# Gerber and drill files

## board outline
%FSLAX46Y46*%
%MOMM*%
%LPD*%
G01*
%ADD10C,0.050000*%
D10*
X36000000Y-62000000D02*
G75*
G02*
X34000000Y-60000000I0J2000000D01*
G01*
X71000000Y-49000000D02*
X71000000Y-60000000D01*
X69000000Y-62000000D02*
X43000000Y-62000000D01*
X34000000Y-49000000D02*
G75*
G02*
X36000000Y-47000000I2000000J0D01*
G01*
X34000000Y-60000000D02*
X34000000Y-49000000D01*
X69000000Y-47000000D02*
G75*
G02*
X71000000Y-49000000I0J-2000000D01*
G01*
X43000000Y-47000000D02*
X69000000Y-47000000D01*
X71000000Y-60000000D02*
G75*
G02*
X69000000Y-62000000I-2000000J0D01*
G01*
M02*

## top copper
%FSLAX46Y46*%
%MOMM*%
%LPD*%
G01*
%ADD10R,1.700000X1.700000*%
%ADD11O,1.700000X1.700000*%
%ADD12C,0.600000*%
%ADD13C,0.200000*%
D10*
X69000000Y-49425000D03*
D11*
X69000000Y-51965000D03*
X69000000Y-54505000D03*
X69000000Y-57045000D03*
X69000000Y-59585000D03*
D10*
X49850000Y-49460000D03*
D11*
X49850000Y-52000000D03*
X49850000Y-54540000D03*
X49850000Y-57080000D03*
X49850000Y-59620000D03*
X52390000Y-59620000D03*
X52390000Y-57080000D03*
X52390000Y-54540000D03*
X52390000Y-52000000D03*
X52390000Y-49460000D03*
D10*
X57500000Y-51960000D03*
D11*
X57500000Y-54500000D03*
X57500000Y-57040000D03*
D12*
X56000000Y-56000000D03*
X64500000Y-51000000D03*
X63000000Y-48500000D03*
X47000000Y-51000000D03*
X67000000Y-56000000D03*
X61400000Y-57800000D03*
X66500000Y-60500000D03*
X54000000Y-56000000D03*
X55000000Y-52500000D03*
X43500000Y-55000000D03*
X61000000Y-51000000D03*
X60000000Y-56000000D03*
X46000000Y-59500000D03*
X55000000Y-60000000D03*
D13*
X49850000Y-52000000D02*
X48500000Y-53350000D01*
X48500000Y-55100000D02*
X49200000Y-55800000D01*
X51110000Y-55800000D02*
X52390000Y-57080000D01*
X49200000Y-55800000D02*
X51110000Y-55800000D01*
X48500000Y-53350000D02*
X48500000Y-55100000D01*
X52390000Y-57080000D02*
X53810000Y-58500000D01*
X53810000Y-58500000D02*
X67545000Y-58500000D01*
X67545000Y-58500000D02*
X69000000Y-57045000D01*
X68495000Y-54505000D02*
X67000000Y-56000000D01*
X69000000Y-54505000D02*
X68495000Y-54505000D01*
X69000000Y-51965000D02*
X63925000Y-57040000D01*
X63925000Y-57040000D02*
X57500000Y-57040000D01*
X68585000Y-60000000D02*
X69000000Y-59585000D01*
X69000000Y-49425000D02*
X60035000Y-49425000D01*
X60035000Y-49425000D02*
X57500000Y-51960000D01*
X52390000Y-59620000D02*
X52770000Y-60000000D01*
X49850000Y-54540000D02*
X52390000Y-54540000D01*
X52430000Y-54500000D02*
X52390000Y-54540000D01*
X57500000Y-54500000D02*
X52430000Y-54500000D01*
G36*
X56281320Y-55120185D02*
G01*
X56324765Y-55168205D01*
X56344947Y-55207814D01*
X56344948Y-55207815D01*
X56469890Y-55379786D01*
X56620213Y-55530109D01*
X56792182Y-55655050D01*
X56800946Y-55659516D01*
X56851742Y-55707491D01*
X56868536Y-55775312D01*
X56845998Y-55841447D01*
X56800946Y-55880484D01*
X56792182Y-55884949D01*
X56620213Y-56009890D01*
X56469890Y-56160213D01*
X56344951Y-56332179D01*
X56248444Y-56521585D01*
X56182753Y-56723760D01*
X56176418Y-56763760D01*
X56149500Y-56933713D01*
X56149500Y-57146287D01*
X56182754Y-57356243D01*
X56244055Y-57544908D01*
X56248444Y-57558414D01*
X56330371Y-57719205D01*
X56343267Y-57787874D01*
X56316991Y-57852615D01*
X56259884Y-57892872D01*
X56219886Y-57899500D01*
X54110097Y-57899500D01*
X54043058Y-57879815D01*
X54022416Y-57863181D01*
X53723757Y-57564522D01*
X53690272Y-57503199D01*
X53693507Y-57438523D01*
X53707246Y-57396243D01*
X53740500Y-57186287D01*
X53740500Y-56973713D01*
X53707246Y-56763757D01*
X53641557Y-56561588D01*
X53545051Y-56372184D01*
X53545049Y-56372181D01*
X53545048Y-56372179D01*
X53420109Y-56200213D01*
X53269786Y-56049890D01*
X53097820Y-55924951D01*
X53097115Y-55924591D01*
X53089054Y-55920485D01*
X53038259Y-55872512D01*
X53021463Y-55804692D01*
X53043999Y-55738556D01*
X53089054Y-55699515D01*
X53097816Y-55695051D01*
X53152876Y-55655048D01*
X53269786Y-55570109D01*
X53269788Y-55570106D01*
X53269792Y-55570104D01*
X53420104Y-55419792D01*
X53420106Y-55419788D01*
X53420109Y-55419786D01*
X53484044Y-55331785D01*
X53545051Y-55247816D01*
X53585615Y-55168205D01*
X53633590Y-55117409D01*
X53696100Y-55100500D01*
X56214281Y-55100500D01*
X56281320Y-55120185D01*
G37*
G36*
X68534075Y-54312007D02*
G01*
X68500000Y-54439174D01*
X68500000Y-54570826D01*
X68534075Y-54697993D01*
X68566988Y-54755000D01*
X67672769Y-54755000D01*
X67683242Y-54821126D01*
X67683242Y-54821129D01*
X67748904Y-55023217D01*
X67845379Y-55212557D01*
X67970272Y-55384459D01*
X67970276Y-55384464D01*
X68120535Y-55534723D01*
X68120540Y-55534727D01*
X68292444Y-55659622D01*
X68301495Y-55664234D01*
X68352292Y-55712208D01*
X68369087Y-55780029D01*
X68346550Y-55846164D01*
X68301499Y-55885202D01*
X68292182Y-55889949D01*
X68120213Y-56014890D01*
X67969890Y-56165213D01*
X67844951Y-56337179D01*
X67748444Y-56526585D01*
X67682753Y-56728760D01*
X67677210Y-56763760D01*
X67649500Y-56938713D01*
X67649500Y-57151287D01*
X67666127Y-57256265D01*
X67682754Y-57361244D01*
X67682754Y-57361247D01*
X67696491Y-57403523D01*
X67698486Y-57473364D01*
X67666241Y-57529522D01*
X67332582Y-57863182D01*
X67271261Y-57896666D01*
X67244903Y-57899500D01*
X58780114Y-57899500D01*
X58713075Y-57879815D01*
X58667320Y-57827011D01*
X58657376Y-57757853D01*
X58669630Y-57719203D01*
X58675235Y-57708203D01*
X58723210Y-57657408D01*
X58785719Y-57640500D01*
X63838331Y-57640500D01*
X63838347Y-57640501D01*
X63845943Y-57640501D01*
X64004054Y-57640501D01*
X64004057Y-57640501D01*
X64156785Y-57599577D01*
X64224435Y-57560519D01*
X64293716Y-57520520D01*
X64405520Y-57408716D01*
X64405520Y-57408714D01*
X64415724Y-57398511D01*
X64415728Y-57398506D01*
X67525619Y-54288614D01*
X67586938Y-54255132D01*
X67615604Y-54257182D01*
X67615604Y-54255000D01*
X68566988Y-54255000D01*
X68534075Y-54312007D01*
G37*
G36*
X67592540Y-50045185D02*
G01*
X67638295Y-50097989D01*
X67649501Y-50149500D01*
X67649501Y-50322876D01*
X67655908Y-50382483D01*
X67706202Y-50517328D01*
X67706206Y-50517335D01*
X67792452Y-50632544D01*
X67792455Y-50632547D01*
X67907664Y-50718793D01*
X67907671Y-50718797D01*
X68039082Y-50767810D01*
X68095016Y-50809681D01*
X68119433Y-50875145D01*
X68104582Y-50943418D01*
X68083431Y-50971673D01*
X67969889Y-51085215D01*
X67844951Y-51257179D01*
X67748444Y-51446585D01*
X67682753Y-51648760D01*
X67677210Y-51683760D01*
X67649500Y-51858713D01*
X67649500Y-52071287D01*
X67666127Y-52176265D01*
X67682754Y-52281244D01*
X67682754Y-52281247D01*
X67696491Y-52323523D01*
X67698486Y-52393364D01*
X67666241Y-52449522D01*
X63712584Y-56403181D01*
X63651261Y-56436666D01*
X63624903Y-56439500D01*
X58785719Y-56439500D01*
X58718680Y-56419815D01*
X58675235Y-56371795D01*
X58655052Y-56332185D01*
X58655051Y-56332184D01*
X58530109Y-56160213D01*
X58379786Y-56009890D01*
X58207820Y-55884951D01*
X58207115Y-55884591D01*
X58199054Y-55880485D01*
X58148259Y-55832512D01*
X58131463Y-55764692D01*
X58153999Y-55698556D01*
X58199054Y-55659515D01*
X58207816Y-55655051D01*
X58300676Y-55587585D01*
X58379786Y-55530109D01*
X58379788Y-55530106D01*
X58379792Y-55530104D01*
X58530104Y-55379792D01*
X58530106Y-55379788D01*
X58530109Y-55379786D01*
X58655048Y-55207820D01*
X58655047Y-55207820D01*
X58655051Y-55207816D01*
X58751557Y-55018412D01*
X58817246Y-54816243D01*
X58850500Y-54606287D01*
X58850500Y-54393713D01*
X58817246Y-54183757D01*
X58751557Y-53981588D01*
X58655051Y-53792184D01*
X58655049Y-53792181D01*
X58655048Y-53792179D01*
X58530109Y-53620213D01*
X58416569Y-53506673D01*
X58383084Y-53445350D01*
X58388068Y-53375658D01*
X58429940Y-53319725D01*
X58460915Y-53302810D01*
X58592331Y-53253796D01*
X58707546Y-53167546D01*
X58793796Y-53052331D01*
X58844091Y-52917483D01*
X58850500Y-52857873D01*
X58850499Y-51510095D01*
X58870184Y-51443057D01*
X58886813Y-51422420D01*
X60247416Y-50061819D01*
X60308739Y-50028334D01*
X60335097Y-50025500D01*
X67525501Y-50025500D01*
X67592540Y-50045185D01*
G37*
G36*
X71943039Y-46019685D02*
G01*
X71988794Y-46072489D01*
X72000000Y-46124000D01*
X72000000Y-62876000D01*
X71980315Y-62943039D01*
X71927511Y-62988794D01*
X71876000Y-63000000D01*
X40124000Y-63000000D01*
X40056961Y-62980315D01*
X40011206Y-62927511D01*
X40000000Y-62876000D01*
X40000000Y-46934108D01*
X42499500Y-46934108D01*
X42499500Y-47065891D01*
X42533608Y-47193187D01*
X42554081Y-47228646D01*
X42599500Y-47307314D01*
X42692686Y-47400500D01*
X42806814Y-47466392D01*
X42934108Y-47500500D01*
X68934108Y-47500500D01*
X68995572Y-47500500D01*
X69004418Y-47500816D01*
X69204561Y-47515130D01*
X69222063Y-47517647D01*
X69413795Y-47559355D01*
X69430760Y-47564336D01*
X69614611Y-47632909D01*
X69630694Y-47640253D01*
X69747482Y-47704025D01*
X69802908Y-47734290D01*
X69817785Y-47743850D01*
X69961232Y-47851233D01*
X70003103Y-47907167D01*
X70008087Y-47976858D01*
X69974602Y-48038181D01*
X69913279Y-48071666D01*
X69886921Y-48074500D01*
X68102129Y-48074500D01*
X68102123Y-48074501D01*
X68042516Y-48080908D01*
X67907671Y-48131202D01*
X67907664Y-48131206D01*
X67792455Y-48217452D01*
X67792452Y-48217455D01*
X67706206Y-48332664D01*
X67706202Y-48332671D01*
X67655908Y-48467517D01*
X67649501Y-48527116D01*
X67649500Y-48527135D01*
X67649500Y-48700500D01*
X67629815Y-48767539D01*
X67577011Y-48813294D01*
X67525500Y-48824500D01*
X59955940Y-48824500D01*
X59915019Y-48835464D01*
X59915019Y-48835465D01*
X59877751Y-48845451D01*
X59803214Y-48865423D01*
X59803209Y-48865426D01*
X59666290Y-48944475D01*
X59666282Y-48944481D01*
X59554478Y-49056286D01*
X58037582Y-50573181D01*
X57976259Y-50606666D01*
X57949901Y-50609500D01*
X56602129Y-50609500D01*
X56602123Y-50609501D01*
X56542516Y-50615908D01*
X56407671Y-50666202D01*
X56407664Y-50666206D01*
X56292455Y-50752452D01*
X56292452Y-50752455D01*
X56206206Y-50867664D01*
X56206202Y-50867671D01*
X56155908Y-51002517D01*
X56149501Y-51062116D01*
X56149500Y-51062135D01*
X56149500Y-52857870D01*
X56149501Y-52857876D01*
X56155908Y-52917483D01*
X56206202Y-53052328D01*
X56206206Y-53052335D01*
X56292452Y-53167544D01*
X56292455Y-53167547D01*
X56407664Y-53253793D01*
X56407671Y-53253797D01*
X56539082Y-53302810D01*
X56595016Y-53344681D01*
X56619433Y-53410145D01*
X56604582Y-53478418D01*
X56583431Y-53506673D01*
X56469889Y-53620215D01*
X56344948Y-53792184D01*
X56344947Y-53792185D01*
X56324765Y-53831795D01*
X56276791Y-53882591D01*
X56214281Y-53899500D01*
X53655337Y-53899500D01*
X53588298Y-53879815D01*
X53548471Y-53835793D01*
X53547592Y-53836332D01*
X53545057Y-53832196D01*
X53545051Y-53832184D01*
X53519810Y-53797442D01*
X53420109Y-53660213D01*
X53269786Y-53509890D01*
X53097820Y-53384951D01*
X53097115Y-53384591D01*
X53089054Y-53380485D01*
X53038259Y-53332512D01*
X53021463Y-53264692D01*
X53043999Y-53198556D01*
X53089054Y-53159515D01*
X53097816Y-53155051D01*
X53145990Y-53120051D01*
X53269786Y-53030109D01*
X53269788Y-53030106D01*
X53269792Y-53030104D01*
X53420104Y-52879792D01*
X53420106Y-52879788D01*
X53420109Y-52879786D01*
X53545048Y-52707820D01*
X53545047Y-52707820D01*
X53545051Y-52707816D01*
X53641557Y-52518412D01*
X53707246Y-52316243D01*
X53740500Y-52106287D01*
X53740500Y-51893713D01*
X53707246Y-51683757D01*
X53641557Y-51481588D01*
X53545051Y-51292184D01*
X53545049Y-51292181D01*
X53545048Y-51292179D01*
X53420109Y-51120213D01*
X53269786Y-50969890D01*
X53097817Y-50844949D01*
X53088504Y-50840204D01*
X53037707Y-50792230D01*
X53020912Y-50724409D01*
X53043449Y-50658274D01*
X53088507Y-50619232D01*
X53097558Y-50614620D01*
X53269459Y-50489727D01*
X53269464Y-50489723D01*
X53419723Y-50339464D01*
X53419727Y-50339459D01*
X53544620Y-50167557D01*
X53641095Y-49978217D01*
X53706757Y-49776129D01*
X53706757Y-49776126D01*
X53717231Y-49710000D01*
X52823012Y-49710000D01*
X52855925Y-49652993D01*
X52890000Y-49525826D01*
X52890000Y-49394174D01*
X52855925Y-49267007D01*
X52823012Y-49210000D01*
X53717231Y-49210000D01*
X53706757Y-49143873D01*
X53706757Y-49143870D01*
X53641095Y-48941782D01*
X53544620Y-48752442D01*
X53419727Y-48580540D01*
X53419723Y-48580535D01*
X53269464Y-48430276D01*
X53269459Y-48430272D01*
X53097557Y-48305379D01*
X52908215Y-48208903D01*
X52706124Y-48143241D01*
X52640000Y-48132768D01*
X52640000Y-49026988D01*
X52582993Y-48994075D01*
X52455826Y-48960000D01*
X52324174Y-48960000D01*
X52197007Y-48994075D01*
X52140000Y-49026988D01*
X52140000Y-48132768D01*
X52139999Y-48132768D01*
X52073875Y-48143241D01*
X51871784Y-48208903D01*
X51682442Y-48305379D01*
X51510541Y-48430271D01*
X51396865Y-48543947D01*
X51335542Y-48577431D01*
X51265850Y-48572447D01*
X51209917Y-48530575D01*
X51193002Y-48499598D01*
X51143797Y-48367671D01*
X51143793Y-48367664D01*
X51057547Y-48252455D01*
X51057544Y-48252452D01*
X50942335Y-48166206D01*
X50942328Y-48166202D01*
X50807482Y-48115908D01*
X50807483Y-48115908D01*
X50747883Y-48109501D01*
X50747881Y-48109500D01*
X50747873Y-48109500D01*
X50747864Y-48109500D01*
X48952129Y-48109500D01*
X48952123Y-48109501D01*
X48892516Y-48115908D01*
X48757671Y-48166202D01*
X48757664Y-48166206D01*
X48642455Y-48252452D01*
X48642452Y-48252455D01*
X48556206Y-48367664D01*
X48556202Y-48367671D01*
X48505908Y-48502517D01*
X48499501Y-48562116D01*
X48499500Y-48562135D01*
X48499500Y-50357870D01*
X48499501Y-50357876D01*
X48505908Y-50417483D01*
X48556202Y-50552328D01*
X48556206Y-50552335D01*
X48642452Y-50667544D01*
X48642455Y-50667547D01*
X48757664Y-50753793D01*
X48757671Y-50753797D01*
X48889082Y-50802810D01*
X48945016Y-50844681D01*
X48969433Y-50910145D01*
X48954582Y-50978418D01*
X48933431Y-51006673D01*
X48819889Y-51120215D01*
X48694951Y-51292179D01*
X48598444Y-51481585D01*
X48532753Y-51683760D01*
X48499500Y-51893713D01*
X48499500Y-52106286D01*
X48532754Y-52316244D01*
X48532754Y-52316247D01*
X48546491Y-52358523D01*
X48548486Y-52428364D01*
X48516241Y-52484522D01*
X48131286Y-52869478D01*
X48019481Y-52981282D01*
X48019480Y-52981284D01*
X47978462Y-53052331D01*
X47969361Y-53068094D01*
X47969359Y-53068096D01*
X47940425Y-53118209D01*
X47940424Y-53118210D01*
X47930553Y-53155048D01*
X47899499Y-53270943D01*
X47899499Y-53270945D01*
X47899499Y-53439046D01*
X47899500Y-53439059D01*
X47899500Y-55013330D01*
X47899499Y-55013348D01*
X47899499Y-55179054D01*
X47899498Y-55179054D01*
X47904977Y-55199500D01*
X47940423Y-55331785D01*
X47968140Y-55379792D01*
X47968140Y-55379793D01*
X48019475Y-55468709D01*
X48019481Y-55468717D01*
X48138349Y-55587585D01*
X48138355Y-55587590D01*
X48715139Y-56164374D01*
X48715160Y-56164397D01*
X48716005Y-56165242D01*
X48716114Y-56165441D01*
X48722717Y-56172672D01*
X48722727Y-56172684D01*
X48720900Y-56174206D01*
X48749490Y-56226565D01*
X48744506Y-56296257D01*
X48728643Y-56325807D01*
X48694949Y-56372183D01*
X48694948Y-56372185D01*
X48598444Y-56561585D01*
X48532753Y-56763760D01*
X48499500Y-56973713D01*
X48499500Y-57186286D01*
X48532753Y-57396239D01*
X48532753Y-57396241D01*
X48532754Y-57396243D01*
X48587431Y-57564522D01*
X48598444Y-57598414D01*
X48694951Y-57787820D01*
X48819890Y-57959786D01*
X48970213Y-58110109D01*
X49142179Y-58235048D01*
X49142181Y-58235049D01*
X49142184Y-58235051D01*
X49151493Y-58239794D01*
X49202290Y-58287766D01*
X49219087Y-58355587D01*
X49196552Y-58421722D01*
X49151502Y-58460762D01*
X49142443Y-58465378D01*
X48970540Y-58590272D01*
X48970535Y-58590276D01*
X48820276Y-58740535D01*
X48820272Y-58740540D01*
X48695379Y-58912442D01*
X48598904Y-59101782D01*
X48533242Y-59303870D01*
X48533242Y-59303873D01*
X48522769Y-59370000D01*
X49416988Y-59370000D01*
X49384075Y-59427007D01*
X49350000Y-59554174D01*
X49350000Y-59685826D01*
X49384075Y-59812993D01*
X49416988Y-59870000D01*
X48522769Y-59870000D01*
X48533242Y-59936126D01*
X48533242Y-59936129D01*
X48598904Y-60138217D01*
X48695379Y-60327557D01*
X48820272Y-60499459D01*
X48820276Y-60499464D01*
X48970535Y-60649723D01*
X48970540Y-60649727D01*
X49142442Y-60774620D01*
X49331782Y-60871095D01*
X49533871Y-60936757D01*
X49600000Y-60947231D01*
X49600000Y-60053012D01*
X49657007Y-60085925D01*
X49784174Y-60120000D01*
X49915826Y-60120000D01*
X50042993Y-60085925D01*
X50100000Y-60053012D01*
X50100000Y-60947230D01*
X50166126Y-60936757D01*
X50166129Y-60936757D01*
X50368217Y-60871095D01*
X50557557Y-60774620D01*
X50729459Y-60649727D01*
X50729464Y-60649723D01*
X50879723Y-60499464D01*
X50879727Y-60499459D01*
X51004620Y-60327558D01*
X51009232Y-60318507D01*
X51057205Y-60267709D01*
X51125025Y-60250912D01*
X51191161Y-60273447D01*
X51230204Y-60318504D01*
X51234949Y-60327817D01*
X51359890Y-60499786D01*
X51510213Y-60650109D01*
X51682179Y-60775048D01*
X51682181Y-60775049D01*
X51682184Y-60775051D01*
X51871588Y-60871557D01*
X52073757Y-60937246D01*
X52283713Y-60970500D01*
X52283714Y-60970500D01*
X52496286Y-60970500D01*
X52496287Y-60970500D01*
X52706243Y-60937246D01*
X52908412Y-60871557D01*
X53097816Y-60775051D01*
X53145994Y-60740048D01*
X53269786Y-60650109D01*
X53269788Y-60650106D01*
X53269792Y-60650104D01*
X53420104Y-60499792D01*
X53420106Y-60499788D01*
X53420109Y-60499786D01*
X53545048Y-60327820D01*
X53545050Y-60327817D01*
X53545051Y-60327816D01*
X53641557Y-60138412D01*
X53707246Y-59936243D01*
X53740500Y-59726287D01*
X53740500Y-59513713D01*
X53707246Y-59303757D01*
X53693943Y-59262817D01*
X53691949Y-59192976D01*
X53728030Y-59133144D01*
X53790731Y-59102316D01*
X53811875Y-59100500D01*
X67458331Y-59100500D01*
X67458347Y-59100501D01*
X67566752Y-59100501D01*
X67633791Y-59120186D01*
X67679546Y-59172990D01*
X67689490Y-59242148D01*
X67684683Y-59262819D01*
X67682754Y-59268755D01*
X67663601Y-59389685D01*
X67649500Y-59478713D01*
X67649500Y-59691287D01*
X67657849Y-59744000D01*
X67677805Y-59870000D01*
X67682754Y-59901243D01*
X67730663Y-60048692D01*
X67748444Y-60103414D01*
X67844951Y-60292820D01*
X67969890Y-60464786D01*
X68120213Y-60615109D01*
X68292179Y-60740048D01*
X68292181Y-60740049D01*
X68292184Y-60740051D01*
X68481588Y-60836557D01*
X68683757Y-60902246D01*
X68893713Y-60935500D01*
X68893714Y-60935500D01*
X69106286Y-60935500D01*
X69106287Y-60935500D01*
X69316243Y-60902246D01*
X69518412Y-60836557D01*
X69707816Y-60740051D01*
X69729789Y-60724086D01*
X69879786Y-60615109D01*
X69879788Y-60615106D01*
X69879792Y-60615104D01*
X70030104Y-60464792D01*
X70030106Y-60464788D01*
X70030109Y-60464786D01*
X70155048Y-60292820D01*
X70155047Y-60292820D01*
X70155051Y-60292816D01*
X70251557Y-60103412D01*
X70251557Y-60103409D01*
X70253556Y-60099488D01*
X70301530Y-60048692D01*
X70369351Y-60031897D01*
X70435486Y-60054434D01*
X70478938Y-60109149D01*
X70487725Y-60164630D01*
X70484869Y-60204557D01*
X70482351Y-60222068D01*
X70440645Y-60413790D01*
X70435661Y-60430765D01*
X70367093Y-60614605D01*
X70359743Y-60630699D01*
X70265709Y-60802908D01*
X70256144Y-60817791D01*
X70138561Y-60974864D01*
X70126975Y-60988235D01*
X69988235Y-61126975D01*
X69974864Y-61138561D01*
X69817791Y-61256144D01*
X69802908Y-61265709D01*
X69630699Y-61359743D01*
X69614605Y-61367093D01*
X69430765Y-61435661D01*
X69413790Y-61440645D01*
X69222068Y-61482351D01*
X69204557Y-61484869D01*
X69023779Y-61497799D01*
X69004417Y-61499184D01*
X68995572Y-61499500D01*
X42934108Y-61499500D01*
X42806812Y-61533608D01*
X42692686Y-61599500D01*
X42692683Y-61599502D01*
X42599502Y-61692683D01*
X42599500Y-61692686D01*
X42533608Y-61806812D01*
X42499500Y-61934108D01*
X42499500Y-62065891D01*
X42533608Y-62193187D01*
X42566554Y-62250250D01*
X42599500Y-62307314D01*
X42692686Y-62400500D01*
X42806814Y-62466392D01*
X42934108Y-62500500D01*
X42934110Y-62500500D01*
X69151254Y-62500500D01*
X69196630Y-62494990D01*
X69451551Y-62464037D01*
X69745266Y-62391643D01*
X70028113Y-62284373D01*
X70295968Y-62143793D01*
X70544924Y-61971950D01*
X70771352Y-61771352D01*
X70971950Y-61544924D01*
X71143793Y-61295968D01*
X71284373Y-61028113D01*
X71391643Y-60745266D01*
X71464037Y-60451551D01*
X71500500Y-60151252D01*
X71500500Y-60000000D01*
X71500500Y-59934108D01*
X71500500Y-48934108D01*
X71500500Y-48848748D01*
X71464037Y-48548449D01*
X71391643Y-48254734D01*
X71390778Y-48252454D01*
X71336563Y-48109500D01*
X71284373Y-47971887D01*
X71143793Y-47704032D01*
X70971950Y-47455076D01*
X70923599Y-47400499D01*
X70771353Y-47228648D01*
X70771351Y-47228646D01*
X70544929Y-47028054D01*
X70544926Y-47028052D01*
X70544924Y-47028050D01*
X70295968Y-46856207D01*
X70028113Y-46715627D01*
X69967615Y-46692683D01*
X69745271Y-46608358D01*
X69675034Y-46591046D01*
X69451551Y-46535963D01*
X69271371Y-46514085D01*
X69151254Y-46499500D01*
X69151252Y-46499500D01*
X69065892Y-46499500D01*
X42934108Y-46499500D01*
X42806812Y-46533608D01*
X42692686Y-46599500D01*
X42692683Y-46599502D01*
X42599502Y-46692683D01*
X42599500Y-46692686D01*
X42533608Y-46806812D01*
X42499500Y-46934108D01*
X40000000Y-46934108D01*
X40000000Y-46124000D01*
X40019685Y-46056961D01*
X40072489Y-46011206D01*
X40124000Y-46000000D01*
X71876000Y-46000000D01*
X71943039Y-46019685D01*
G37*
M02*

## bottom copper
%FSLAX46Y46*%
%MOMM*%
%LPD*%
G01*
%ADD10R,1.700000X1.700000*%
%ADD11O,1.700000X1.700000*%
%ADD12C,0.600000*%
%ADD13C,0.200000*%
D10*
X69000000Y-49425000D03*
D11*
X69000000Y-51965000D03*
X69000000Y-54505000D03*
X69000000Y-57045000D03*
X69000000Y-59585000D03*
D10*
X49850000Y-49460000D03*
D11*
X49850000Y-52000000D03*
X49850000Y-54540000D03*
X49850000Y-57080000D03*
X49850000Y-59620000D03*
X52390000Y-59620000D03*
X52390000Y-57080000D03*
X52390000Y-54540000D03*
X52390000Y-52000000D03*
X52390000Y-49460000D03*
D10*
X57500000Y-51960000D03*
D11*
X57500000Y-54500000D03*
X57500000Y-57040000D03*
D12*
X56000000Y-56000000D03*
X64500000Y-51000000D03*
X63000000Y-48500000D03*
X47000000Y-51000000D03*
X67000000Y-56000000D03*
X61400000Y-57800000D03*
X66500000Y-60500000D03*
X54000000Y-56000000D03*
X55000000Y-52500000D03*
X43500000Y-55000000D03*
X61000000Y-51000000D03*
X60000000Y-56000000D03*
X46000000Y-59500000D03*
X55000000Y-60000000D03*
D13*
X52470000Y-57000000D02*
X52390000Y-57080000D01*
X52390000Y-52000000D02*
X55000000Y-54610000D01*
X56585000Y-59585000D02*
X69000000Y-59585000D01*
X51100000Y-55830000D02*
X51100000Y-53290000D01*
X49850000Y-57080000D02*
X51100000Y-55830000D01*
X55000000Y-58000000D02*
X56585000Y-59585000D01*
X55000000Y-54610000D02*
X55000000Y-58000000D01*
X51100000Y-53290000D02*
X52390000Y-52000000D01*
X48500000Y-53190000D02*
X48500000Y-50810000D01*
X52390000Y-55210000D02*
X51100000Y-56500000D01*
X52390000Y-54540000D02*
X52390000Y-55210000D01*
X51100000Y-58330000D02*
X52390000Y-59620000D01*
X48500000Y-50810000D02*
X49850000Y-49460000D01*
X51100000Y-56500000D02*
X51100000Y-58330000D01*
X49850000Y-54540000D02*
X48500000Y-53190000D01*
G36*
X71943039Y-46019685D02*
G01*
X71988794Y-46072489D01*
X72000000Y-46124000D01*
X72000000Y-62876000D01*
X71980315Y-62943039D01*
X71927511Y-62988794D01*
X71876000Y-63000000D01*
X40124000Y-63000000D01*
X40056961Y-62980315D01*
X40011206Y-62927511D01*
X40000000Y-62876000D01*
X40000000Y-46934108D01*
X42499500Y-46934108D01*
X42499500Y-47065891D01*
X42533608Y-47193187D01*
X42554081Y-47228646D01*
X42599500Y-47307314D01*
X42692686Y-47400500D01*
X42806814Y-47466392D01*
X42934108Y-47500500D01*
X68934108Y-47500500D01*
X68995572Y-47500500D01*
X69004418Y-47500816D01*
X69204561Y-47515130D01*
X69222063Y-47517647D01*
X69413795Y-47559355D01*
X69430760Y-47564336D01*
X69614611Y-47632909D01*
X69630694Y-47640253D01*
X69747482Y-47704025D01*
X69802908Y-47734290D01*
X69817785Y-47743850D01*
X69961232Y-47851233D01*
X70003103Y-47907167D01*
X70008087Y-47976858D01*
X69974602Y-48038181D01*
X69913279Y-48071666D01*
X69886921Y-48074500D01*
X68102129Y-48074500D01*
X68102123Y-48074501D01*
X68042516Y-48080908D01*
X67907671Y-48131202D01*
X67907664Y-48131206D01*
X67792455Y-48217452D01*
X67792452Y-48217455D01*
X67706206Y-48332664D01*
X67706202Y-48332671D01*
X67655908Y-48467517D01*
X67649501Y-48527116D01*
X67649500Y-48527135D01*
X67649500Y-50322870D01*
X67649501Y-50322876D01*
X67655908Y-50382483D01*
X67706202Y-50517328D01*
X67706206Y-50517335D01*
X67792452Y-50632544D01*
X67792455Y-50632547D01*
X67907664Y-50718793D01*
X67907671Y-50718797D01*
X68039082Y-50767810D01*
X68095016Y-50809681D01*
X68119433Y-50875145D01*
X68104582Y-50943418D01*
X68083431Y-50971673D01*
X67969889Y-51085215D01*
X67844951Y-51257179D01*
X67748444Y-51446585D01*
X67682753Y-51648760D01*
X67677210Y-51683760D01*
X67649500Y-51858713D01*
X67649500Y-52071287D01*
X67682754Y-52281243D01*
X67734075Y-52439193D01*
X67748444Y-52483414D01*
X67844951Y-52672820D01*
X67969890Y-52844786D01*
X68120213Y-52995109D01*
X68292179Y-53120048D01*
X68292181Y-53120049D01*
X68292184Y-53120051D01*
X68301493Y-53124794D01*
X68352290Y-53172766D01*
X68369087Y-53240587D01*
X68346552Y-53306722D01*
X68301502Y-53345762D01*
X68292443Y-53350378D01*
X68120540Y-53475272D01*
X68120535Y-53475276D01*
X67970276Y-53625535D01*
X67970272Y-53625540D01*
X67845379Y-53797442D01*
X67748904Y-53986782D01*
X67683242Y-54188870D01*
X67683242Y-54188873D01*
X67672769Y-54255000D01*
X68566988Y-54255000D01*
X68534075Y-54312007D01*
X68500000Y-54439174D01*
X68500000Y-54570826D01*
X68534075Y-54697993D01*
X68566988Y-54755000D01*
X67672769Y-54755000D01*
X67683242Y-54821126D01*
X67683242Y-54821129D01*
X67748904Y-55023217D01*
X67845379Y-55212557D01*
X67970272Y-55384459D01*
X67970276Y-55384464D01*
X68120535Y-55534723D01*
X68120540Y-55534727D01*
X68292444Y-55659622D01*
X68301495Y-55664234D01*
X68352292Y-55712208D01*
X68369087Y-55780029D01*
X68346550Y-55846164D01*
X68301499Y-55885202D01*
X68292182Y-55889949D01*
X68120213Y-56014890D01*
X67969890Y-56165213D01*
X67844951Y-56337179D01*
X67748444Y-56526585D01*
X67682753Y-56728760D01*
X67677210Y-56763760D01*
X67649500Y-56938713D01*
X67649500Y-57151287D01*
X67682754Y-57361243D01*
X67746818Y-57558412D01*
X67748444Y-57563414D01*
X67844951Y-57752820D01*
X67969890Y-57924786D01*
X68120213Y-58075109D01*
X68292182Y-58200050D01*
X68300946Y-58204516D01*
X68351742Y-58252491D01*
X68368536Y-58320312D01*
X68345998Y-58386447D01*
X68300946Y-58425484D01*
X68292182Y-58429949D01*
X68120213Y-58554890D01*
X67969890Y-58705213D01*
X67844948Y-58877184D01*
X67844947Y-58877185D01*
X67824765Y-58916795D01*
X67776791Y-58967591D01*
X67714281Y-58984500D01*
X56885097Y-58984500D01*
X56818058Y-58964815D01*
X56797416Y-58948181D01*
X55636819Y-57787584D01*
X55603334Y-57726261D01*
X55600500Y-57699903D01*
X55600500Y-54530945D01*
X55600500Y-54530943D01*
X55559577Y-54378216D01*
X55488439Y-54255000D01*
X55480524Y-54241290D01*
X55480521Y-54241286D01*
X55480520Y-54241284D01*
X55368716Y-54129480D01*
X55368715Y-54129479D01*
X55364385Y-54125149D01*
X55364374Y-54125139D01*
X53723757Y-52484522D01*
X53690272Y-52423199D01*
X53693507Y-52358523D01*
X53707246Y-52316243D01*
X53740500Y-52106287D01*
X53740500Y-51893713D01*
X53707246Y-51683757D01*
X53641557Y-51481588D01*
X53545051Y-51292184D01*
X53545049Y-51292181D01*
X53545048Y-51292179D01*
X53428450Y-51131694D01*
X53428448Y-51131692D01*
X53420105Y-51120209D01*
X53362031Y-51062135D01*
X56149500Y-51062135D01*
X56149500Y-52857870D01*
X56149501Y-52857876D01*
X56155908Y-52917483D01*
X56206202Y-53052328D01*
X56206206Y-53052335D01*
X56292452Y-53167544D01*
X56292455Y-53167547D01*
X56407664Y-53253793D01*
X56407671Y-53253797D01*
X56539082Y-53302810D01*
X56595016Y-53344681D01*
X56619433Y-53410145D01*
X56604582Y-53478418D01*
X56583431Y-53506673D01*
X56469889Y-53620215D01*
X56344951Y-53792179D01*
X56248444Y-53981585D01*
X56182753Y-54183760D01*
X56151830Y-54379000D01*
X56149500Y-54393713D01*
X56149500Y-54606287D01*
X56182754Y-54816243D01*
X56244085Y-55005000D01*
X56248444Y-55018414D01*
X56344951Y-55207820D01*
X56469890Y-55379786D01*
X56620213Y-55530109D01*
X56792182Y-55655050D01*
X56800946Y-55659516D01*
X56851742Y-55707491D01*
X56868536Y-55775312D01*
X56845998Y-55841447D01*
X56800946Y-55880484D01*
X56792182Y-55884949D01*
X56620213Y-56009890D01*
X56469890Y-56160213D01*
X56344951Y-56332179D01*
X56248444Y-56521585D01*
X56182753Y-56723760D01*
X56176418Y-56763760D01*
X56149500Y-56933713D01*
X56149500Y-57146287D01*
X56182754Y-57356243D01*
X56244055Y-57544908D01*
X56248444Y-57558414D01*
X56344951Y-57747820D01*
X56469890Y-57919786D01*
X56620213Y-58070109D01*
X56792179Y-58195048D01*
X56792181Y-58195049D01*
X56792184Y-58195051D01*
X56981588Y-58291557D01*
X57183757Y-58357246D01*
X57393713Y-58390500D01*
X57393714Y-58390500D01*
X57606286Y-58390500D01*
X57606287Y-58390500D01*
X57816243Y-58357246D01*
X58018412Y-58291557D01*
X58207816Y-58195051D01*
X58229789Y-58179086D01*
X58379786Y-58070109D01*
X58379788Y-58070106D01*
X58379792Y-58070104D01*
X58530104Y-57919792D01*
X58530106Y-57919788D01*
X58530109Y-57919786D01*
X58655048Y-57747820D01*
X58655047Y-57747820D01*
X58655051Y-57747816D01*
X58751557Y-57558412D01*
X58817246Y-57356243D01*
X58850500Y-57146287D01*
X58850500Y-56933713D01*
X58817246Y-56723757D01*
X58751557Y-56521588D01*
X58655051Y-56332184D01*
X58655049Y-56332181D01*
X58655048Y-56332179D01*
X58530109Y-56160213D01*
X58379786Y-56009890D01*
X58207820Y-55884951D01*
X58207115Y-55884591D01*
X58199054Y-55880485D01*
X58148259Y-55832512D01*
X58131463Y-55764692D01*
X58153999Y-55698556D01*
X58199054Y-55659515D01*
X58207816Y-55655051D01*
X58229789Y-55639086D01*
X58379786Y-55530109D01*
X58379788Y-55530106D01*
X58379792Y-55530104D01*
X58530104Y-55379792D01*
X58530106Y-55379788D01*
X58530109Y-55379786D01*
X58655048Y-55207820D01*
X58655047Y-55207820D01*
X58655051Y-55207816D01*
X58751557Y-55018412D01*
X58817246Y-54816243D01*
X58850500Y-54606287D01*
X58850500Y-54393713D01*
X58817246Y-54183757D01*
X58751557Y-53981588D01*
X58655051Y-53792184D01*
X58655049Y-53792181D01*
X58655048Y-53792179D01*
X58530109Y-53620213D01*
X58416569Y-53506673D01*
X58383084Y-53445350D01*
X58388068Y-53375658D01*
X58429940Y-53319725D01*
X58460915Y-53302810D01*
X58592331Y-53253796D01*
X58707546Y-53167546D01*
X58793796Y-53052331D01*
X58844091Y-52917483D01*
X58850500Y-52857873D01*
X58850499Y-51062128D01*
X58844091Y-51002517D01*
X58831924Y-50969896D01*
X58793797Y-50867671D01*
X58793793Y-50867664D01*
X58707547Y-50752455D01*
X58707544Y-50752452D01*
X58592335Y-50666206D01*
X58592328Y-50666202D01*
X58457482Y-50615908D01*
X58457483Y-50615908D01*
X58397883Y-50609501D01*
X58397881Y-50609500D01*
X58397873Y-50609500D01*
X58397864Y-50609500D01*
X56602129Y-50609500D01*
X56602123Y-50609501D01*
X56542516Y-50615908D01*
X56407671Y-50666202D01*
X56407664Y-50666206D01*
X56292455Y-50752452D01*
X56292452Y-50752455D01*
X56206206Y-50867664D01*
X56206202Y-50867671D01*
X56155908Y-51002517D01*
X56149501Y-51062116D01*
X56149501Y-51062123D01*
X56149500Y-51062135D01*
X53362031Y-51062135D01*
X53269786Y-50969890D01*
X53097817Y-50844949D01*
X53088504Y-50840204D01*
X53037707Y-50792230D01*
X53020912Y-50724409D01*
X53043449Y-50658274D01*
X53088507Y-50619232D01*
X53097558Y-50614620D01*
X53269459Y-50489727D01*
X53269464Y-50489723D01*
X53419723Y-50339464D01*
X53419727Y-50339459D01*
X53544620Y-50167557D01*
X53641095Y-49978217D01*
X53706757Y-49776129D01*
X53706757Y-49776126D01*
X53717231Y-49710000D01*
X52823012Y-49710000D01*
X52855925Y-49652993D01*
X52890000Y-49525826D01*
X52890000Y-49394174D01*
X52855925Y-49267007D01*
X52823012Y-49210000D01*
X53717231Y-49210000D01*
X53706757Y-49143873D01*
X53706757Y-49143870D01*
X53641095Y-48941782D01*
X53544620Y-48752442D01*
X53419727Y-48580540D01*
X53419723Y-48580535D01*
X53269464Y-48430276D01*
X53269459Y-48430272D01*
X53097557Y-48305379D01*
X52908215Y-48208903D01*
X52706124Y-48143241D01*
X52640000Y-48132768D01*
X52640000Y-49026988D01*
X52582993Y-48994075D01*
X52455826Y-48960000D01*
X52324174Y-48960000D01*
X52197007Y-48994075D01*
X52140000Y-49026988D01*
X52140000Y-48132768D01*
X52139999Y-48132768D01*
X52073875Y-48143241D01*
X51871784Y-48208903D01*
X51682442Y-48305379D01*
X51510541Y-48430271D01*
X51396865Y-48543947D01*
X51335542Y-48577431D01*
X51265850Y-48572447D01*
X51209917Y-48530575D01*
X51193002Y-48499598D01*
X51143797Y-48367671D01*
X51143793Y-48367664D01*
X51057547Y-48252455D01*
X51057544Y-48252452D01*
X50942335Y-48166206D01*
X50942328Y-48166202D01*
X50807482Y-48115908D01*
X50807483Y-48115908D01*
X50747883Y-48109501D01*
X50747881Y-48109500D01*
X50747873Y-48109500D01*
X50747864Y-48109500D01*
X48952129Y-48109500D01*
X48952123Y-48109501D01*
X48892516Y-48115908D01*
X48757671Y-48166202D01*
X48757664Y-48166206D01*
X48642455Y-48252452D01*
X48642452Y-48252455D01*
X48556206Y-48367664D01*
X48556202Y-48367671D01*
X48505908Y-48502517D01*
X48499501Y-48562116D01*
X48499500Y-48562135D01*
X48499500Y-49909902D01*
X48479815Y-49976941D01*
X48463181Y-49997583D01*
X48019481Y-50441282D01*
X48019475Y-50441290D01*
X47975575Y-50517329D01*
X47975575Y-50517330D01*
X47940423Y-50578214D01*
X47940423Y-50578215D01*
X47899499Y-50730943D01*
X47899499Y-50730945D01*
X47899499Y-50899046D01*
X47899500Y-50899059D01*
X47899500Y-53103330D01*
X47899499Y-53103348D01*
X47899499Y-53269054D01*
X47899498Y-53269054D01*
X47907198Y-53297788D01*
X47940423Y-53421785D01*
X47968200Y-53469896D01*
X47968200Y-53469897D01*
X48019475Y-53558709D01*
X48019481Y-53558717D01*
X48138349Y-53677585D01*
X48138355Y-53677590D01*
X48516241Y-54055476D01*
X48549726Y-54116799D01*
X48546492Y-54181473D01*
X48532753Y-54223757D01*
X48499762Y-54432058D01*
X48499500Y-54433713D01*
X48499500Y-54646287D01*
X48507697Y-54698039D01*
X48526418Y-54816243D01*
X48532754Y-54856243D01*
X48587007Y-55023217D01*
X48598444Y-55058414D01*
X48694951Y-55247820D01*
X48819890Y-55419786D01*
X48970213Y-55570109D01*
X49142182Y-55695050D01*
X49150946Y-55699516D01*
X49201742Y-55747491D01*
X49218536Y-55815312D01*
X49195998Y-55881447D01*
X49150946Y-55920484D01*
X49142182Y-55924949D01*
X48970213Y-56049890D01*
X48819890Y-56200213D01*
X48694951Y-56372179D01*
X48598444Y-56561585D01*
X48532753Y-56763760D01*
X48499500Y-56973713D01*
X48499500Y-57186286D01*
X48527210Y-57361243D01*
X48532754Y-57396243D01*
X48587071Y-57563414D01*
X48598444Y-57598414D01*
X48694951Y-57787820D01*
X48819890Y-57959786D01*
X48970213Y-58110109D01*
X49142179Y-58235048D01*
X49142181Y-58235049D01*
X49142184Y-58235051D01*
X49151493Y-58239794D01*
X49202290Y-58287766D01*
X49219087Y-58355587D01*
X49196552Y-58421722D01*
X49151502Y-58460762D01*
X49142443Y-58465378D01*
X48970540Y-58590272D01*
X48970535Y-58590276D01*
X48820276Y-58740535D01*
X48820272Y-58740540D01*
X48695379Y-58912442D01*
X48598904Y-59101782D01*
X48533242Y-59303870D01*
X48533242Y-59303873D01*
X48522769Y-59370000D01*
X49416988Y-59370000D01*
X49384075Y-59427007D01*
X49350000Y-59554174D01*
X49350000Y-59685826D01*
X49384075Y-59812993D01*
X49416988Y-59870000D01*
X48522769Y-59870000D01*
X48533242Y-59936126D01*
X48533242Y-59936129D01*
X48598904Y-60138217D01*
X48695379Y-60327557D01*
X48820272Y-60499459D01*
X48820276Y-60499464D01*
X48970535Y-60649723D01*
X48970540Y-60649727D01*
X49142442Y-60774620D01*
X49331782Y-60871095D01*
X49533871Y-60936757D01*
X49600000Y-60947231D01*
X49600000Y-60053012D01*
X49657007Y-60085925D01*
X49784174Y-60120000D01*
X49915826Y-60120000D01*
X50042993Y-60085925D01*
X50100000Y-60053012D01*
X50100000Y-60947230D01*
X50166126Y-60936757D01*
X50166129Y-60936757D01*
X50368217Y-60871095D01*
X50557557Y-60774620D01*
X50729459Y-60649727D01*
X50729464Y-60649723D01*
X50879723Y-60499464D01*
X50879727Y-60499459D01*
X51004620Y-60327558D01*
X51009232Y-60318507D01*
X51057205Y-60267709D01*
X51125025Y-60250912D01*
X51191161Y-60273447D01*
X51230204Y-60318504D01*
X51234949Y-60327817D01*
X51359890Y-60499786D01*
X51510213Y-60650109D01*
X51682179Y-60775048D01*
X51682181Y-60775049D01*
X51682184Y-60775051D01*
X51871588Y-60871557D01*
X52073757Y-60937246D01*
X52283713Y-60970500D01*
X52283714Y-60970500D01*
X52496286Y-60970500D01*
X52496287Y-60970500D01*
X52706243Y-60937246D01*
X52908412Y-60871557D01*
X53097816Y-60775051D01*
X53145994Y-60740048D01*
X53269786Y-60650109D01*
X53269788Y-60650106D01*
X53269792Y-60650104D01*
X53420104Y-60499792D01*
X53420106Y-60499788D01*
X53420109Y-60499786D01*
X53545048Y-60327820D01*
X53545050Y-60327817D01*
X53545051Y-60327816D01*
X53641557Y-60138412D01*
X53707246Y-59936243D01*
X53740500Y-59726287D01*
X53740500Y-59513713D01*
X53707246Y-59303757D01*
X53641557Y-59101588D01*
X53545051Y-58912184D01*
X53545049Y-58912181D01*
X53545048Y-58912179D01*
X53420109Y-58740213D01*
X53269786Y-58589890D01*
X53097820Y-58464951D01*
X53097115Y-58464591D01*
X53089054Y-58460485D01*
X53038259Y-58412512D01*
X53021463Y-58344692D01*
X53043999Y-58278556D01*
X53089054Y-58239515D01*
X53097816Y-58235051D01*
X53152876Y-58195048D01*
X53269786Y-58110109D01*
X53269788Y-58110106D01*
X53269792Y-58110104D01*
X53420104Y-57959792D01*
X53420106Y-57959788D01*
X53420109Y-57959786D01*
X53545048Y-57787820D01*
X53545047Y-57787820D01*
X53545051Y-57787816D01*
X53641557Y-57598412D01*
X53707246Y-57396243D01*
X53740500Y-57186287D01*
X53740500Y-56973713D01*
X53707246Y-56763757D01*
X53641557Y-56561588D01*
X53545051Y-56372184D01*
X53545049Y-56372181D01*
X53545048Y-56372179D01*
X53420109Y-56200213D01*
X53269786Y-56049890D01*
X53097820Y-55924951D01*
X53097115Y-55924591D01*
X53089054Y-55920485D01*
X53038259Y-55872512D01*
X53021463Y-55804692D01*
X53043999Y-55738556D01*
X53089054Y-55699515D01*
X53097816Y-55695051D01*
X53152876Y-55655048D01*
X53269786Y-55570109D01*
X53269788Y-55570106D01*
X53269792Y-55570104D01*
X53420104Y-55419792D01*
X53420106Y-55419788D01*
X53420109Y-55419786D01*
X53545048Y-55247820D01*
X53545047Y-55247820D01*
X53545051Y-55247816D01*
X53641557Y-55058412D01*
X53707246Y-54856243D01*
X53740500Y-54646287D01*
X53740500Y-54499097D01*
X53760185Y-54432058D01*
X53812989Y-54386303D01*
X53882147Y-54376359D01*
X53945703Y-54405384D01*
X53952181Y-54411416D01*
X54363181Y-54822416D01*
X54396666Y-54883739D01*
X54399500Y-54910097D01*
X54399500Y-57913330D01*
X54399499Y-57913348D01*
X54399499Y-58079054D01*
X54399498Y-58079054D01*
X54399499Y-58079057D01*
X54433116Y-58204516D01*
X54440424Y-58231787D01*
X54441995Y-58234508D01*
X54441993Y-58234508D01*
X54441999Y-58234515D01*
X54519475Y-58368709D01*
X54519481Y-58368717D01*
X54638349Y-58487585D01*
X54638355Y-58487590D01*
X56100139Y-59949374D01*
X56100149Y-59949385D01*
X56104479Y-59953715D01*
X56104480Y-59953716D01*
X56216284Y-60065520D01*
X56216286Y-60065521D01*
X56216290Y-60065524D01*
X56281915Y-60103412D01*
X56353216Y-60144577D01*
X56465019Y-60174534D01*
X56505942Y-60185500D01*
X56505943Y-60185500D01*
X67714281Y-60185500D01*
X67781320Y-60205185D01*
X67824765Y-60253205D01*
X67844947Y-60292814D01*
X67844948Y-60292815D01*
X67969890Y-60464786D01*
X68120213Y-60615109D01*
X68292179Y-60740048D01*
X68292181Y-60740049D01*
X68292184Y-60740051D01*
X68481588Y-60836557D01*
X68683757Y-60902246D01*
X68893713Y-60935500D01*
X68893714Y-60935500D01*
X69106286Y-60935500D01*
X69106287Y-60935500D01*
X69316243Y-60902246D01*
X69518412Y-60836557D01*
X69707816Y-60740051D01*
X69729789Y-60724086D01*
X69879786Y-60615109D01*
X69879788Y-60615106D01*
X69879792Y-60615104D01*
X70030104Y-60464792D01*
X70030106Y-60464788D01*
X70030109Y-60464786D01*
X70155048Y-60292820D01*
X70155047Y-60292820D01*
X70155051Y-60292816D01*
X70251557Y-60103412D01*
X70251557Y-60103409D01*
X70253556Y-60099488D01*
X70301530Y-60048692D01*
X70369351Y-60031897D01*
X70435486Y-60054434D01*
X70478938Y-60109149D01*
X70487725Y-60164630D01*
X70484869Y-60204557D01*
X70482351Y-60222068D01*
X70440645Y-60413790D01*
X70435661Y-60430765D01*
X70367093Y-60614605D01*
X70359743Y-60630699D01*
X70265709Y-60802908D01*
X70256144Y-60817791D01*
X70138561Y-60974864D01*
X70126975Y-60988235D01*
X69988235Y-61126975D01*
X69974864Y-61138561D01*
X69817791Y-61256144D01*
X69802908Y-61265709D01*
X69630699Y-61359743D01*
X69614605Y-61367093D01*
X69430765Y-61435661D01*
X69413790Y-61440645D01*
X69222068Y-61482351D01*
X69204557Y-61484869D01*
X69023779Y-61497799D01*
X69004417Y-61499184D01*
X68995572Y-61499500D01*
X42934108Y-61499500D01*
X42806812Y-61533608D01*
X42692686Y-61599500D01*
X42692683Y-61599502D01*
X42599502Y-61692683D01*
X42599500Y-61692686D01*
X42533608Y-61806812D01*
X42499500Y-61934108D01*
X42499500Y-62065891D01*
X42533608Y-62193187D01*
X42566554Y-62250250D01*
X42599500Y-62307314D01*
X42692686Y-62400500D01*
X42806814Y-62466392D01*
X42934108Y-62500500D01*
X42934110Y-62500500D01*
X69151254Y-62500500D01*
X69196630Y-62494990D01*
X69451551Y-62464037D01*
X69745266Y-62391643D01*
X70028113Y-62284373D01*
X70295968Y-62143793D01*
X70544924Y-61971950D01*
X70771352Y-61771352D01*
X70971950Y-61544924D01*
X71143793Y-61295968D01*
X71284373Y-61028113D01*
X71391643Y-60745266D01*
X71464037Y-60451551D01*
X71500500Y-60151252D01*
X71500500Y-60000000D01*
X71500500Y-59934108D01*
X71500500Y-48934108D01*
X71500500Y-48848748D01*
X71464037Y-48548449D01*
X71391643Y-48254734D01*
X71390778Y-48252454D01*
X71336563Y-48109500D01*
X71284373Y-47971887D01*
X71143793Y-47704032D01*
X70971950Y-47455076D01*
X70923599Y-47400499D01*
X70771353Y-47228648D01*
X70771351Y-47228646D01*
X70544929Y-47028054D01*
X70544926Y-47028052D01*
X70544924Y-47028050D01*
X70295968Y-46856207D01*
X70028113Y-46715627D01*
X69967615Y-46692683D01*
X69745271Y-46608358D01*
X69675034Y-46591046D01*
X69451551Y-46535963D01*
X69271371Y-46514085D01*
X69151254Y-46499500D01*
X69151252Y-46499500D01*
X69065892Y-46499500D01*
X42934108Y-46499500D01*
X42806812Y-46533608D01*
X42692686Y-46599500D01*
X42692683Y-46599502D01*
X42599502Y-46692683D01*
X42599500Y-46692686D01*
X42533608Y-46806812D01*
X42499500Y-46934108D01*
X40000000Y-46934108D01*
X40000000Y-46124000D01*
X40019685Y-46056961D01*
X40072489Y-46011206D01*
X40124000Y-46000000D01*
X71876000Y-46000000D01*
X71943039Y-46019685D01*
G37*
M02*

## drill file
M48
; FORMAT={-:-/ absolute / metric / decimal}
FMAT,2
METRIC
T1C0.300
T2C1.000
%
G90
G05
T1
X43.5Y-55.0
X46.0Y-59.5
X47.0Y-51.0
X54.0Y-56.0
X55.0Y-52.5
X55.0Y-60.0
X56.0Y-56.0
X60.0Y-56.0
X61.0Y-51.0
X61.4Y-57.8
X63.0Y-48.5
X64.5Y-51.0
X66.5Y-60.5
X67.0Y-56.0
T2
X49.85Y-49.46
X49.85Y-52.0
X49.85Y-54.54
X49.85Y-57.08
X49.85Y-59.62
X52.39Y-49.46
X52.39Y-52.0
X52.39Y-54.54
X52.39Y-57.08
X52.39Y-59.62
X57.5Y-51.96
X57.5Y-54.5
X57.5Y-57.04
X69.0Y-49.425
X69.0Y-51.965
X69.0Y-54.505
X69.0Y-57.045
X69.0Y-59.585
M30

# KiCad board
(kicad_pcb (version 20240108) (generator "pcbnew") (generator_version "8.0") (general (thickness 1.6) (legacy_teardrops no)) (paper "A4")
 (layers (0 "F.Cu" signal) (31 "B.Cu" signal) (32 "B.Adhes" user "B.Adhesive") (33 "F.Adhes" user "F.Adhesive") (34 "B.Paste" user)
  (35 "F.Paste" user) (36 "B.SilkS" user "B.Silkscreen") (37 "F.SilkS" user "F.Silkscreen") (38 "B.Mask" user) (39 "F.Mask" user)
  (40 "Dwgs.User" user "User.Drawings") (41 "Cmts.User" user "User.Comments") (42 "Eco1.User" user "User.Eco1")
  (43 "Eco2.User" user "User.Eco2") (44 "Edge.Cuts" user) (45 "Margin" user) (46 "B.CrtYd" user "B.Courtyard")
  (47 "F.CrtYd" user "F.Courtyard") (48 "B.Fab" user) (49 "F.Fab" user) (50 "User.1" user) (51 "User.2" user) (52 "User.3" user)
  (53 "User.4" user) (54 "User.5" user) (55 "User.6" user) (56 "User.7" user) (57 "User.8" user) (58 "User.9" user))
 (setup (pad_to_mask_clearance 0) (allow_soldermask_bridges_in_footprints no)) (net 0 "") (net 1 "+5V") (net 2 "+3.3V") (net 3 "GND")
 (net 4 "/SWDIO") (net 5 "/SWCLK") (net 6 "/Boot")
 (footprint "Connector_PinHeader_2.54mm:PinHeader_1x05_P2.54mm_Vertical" (layer "F.Cu") (at 69 49.425)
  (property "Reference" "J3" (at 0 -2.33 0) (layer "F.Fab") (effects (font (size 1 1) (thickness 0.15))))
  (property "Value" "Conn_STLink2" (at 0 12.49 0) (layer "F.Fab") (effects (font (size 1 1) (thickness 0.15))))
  (pad "1" thru_hole rect (at 0 0) (size 1.7 1.7) (drill 1) (layers "*.Cu" "*.Mask") (remove_unused_layers no) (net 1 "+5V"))
  (pad "2" thru_hole oval (at 0 2.54) (size 1.7 1.7) (drill 1) (layers "*.Cu" "*.Mask") (remove_unused_layers no) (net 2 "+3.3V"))
  (pad "3" thru_hole oval (at 0 5.08) (size 1.7 1.7) (drill 1) (layers "*.Cu" "*.Mask") (remove_unused_layers no) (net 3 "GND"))
  (pad "4" thru_hole oval (at 0 7.62) (size 1.7 1.7) (drill 1) (layers "*.Cu" "*.Mask") (remove_unused_layers no) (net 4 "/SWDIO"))
  (pad "5" thru_hole oval (at 0 10.16) (size 1.7 1.7) (drill 1) (layers "*.Cu" "*.Mask") (remove_unused_layers no) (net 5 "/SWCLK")))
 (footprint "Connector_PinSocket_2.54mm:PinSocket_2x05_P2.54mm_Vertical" (layer "F.Cu") (at 52.39 49.46)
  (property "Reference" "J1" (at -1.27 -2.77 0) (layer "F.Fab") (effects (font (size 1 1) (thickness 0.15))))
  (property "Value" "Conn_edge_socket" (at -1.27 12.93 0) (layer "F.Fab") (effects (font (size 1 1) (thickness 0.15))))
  (pad "1" thru_hole rect (at -2.54 0) (size 1.7 1.7) (drill 1) (layers "*.Cu" "*.Mask") (remove_unused_layers no) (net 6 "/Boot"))
  (pad "2" thru_hole oval (at -2.54 2.54) (size 1.7 1.7) (drill 1) (layers "*.Cu" "*.Mask") (remove_unused_layers no) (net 4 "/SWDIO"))
  (pad "3" thru_hole oval (at -2.54 5.08) (size 1.7 1.7) (drill 1) (layers "*.Cu" "*.Mask") (remove_unused_layers no) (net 6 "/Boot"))
  (pad "4" thru_hole oval (at -2.54 7.62) (size 1.7 1.7) (drill 1) (layers "*.Cu" "*.Mask") (remove_unused_layers no) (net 5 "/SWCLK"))
  (pad "5" thru_hole oval (at -2.54 10.16) (size 1.7 1.7) (drill 1) (layers "*.Cu" "*.Mask") (remove_unused_layers no) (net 3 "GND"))
  (pad "6" thru_hole oval (at 0 10.16) (size 1.7 1.7) (drill 1) (layers "*.Cu" "*.Mask") (remove_unused_layers no) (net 6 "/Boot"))
  (pad "7" thru_hole oval (at 0 7.62) (size 1.7 1.7) (drill 1) (layers "*.Cu" "*.Mask") (remove_unused_layers no) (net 4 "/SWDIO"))
  (pad "8" thru_hole oval (at 0 5.08) (size 1.7 1.7) (drill 1) (layers "*.Cu" "*.Mask") (remove_unused_layers no) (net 6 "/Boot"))
  (pad "9" thru_hole oval (at 0 2.54) (size 1.7 1.7) (drill 1) (layers "*.Cu" "*.Mask") (remove_unused_layers no) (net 5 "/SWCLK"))
  (pad "10" thru_hole oval (at 0 0) (size 1.7 1.7) (drill 1) (layers "*.Cu" "*.Mask") (remove_unused_layers no) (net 3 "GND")))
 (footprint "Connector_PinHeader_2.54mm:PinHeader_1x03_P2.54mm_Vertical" (layer "F.Cu") (at 57.5 51.96)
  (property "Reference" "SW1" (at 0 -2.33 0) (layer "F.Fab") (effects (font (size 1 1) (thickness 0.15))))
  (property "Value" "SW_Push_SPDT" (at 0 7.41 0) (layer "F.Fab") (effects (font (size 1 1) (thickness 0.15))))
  (pad "1" thru_hole rect (at 0 0) (size 1.7 1.7) (drill 1) (layers "*.Cu" "*.Mask") (remove_unused_layers no) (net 1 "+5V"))
  (pad "2" thru_hole oval (at 0 2.54) (size 1.7 1.7) (drill 1) (layers "*.Cu" "*.Mask") (remove_unused_layers no) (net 6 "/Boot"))
  (pad "3" thru_hole oval (at 0 5.08) (size 1.7 1.7) (drill 1) (layers "*.Cu" "*.Mask") (remove_unused_layers no) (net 2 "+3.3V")))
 (gr_arc (start 36 62) (mid 34.585786 61.414214) (end 34 60) (stroke (width 0.05) (type default)) (layer "Edge.Cuts"))
 (gr_line (start 71 49) (end 71 60) (stroke (width 0.05) (type default)) (layer "Edge.Cuts"))
 (gr_line (start 69 62) (end 43 62) (stroke (width 0.05) (type default)) (layer "Edge.Cuts"))
 (gr_arc (start 34 49) (mid 34.585786 47.585786) (end 36 47) (stroke (width 0.05) (type default)) (layer "Edge.Cuts"))
 (gr_line (start 34 60) (end 34 49) (stroke (width 0.05) (type default)) (layer "Edge.Cuts"))
 (gr_arc (start 69 47) (mid 70.414214 47.585786) (end 71 49) (stroke (width 0.05) (type default)) (layer "Edge.Cuts"))
 (gr_line (start 43 47) (end 69 47) (stroke (width 0.05) (type default)) (layer "Edge.Cuts"))
 (gr_arc (start 71 60) (mid 70.414214 61.414214) (end 69 62) (stroke (width 0.05) (type default)) (layer "Edge.Cuts"))
 (segment (start 49.85 52) (end 48.5 53.35) (width 0.2) (layer "F.Cu") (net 4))
 (segment (start 48.5 55.1) (end 49.2 55.8) (width 0.2) (layer "F.Cu") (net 4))
 (segment (start 51.11 55.8) (end 52.39 57.08) (width 0.2) (layer "F.Cu") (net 4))
 (segment (start 49.2 55.8) (end 51.11 55.8) (width 0.2) (layer "F.Cu") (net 4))
 (segment (start 48.5 53.35) (end 48.5 55.1) (width 0.2) (layer "F.Cu") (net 4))
 (segment (start 52.39 57.08) (end 53.81 58.5) (width 0.2) (layer "F.Cu") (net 4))
 (segment (start 53.81 58.5) (end 67.545 58.5) (width 0.2) (layer "F.Cu") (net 4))
 (segment (start 67.545 58.5) (end 69 57.045) (width 0.2) (layer "F.Cu") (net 4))
 (segment (start 52.47 57) (end 52.39 57.08) (width 0.2) (layer "B.Cu") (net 4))
 (segment (start 68.495 54.505) (end 67 56) (width 0.2) (layer "F.Cu") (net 3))
 (segment (start 69 54.505) (end 68.495 54.505) (width 0.2) (layer "F.Cu") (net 3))
 (via (at 56 56) (size 0.6) (drill 0.3) (layers "F.Cu" "B.Cu") (free yes) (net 3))
 (via (at 64.5 51) (size 0.6) (drill 0.3) (layers "F.Cu" "B.Cu") (free yes) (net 3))
 (via (at 63 48.5) (size 0.6) (drill 0.3) (layers "F.Cu" "B.Cu") (free yes) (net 3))
 (via (at 47 51) (size 0.6) (drill 0.3) (layers "F.Cu" "B.Cu") (free yes) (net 3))
 (via (at 67 56) (size 0.6) (drill 0.3) (layers "F.Cu" "B.Cu") (free yes) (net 3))
 (via (at 61.4 57.8) (size 0.6) (drill 0.3) (layers "F.Cu" "B.Cu") (free yes) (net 3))
 (via (at 66.5 60.5) (size 0.6) (drill 0.3) (layers "F.Cu" "B.Cu") (free yes) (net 3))
 (via (at 54 56) (size 0.6) (drill 0.3) (layers "F.Cu" "B.Cu") (free yes) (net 3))
 (via (at 55 52.5) (size 0.6) (drill 0.3) (layers "F.Cu" "B.Cu") (free yes) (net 3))
 (via (at 43.5 55) (size 0.6) (drill 0.3) (layers "F.Cu" "B.Cu") (free yes) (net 3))
 (via (at 61 51) (size 0.6) (drill 0.3) (layers "F.Cu" "B.Cu") (free yes) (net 3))
 (via (at 60 56) (size 0.6) (drill 0.3) (layers "F.Cu" "B.Cu") (free yes) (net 3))
 (via (at 46 59.5) (size 0.6) (drill 0.3) (layers "F.Cu" "B.Cu") (free yes) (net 3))
 (via (at 55 60) (size 0.6) (drill 0.3) (layers "F.Cu" "B.Cu") (free yes) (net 3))
 (segment (start 69 51.965) (end 63.925 57.04) (width 0.2) (layer "F.Cu") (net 2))
 (segment (start 63.925 57.04) (end 57.5 57.04) (width 0.2) (layer "F.Cu") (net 2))
 (segment (start 68.585 60) (end 69 59.585) (width 0.2) (layer "F.Cu") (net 5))
 (segment (start 52.39 52) (end 55 54.61) (width 0.2) (layer "B.Cu") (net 5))
 (segment (start 56.585 59.585) (end 69 59.585) (width 0.2) (layer "B.Cu") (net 5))
 (segment (start 51.1 55.83) (end 51.1 53.29) (width 0.2) (layer "B.Cu") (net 5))
 (segment (start 49.85 57.08) (end 51.1 55.83) (width 0.2) (layer "B.Cu") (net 5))
 (segment (start 55 58) (end 56.585 59.585) (width 0.2) (layer "B.Cu") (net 5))
 (segment (start 55 54.61) (end 55 58) (width 0.2) (layer "B.Cu") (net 5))
 (segment (start 51.1 53.29) (end 52.39 52) (width 0.2) (layer "B.Cu") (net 5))
 (segment (start 69 49.425) (end 60.035 49.425) (width 0.2) (layer "F.Cu") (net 1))
 (segment (start 60.035 49.425) (end 57.5 51.96) (width 0.2) (layer "F.Cu") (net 1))
 (segment (start 52.39 59.62) (end 52.77 60) (width 0.2) (layer "F.Cu") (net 6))
 (segment (start 49.85 54.54) (end 52.39 54.54) (width 0.2) (layer "F.Cu") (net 6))
 (segment (start 52.43 54.5) (end 52.39 54.54) (width 0.2) (layer "F.Cu") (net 6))
 (segment (start 57.5 54.5) (end 52.43 54.5) (width 0.2) (layer "F.Cu") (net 6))
 (segment (start 48.5 53.19) (end 48.5 50.81) (width 0.2) (layer "B.Cu") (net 6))
 (segment (start 52.39 55.21) (end 51.1 56.5) (width 0.2) (layer "B.Cu") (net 6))
 (segment (start 52.39 54.54) (end 52.39 55.21) (width 0.2) (layer "B.Cu") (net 6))
 (segment (start 51.1 58.33) (end 52.39 59.62) (width 0.2) (layer "B.Cu") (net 6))
 (segment (start 48.5 50.81) (end 49.85 49.46) (width 0.2) (layer "B.Cu") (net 6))
 (segment (start 51.1 56.5) (end 51.1 58.33) (width 0.2) (layer "B.Cu") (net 6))
 (segment (start 49.85 54.54) (end 48.5 53.19) (width 0.2) (layer "B.Cu") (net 6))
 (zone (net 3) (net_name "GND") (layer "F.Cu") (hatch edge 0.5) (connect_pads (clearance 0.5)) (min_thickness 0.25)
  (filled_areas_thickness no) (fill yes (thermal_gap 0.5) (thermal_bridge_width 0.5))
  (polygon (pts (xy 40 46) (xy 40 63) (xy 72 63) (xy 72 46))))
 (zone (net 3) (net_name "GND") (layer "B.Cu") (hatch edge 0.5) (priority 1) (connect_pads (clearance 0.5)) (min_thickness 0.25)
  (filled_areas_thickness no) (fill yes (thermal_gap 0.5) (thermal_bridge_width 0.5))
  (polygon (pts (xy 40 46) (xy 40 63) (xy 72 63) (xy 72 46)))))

